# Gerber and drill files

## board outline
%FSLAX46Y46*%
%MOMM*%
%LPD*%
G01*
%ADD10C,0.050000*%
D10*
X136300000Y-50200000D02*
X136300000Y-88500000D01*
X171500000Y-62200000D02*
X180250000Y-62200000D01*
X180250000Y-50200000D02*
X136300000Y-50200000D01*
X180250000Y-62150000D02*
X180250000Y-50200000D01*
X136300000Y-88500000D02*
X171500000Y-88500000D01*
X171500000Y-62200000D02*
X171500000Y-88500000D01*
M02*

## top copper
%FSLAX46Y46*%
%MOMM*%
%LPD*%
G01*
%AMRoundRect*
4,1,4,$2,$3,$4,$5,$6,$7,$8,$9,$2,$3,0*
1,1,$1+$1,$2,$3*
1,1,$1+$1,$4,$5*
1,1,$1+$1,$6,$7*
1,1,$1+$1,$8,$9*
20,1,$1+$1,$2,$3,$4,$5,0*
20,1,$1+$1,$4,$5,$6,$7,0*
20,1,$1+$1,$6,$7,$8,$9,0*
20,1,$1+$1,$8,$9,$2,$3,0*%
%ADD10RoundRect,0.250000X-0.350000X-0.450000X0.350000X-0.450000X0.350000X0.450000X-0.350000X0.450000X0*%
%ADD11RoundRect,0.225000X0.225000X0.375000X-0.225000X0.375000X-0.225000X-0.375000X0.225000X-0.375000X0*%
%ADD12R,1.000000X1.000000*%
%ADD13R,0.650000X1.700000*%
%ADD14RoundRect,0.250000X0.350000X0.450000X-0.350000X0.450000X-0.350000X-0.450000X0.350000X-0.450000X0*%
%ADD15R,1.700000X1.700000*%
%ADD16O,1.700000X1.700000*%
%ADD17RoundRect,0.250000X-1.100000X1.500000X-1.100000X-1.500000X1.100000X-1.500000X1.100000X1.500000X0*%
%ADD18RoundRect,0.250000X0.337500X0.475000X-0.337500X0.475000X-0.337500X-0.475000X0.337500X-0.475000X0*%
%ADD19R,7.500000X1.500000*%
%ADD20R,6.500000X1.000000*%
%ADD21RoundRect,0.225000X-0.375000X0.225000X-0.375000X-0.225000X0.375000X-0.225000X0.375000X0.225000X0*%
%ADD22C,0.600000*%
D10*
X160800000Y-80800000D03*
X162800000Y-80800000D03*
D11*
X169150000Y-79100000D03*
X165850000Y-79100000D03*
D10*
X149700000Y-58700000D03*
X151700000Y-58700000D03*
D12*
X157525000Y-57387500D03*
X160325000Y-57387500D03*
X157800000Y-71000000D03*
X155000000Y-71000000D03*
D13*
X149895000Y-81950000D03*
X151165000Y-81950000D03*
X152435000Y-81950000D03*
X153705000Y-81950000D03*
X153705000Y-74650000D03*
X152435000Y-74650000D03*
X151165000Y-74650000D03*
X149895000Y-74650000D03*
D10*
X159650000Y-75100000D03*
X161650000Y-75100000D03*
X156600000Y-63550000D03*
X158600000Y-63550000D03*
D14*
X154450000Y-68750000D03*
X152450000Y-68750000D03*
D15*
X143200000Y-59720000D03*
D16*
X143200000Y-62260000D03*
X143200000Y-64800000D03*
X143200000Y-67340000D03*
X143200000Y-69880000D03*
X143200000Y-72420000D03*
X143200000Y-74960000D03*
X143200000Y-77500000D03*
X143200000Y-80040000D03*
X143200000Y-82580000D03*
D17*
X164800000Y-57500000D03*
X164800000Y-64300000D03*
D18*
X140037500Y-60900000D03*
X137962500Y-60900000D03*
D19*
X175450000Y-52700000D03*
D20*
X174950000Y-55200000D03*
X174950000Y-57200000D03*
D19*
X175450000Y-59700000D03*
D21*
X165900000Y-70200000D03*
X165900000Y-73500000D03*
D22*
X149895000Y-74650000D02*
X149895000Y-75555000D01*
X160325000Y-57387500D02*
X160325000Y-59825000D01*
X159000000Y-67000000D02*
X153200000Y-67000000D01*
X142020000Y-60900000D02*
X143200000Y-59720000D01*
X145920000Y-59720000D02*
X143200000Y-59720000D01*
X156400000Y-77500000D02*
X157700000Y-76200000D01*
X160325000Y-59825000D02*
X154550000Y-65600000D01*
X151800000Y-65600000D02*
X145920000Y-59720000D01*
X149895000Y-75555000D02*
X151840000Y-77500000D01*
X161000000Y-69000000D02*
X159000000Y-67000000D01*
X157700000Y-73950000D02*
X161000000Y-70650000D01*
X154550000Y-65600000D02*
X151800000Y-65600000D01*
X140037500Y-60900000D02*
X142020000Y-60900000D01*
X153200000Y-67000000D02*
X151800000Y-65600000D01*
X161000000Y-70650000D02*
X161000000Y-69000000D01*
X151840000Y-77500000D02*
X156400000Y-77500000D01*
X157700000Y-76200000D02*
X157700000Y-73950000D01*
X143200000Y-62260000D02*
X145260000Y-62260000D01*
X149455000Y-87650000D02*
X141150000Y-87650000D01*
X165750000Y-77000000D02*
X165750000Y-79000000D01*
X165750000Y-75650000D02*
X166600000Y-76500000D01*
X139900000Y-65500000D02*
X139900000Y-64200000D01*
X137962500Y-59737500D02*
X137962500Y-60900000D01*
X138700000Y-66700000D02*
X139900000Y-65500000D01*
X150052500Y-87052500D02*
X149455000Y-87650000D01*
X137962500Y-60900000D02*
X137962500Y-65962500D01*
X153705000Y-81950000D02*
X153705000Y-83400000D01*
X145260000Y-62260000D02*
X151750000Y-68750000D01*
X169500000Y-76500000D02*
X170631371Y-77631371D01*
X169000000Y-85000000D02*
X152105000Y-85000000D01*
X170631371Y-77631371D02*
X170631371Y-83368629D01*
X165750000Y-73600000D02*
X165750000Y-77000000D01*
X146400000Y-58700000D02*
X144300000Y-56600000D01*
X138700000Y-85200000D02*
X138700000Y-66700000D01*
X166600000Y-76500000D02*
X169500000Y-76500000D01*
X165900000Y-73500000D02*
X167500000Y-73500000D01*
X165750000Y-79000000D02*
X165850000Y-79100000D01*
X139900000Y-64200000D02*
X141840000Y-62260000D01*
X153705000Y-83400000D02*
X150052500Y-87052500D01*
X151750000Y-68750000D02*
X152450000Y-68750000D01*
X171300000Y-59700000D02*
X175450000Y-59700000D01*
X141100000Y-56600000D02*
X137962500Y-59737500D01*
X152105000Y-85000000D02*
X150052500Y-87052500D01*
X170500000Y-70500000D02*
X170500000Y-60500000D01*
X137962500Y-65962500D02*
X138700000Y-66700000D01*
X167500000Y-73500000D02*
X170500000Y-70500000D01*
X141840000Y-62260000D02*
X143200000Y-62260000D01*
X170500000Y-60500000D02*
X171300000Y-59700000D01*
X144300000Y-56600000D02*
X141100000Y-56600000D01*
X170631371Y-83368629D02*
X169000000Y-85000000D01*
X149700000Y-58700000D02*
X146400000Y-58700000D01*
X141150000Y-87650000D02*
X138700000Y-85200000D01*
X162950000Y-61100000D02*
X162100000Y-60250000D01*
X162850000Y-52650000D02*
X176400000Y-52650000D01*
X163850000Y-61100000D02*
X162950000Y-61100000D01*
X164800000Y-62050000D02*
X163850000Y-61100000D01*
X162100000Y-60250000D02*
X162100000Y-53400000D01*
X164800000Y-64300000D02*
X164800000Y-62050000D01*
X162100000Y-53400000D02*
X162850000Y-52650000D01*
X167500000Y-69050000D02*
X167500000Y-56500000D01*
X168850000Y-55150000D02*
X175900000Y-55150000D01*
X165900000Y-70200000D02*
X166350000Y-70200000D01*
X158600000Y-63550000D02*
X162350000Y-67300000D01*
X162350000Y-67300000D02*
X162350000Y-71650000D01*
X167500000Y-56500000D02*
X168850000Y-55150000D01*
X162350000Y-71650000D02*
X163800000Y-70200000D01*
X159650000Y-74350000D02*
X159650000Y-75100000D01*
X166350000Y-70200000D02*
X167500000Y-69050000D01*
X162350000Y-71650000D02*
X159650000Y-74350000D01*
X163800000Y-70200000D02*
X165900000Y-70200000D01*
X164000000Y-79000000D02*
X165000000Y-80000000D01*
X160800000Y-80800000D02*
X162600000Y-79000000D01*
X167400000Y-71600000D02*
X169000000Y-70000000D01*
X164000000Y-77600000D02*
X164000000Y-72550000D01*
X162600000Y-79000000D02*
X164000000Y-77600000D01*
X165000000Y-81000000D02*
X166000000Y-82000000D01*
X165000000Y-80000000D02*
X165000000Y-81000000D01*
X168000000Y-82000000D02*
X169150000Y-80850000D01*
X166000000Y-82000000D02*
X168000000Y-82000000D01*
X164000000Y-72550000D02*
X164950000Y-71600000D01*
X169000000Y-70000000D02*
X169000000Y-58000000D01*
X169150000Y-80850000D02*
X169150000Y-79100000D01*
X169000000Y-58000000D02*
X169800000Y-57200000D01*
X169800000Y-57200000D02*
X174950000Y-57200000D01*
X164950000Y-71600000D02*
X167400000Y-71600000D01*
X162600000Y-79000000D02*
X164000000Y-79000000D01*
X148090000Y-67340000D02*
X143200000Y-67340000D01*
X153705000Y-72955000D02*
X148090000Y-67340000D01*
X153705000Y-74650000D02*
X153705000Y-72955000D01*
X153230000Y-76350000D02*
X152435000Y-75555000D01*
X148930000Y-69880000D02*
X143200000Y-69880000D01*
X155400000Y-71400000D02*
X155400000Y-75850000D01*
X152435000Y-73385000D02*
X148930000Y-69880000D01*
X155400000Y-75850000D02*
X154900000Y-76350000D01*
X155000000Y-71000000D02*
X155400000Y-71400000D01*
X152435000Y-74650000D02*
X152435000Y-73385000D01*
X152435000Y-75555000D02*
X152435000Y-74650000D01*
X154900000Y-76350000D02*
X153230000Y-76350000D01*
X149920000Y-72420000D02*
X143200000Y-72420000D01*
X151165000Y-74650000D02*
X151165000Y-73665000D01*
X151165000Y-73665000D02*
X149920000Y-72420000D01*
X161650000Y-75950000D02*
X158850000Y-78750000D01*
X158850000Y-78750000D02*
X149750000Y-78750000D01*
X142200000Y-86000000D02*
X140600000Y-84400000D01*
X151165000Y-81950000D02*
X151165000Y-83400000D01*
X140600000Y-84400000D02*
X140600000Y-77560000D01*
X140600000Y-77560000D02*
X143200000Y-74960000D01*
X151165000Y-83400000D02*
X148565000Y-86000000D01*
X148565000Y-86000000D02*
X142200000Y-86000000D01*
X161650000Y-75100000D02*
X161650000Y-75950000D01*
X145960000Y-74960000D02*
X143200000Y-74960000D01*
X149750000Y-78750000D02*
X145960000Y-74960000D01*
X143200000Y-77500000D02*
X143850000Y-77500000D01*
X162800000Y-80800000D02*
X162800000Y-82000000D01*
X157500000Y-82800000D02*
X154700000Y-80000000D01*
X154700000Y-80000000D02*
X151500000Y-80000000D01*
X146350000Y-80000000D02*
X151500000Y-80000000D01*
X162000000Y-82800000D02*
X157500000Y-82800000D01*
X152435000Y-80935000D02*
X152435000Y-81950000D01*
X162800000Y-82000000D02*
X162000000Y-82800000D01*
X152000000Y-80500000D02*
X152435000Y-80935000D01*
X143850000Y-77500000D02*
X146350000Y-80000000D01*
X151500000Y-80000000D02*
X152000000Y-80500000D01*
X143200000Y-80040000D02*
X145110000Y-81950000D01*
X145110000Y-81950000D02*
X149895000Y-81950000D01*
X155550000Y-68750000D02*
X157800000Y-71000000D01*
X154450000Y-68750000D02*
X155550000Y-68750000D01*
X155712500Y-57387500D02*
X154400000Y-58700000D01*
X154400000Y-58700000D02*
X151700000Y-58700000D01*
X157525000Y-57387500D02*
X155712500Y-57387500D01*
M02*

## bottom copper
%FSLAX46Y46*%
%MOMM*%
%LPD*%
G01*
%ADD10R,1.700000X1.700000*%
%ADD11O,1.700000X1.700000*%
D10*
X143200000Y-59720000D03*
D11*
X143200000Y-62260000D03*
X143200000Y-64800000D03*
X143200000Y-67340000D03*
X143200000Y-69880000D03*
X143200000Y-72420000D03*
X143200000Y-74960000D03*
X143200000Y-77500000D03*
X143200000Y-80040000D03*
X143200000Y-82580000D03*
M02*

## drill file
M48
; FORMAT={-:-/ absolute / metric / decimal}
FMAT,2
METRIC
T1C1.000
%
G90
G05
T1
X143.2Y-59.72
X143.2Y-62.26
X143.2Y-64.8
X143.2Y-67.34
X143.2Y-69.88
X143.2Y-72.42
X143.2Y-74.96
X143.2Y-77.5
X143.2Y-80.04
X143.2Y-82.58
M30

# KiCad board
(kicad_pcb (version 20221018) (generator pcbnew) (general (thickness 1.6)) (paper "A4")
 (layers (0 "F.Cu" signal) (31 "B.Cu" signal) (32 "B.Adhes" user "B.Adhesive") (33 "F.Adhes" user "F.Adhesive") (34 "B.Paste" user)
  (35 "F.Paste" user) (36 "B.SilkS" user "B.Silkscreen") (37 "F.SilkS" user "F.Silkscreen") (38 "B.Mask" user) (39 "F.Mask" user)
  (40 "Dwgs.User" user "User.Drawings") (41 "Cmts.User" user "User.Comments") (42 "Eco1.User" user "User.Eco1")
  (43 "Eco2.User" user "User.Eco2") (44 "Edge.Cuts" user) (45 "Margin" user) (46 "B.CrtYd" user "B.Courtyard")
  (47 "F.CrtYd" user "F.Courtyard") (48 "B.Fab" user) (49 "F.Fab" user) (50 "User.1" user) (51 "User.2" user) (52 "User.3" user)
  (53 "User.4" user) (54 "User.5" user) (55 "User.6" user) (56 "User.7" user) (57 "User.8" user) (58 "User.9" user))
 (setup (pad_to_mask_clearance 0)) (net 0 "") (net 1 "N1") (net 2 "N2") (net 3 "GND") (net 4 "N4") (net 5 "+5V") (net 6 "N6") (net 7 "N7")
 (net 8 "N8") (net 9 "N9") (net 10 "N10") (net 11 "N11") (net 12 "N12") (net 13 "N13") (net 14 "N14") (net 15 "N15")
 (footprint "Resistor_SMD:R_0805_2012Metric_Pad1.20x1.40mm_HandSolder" (layer "F.Cu") (at 161.8 80.8)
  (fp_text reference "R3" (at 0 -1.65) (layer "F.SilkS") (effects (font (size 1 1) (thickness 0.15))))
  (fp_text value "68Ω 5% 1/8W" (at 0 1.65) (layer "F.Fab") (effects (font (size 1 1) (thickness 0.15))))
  (pad "1" smd roundrect (at -1 0) (size 1.2 1.4) (layers "F.Cu" "F.Paste" "F.Mask") (roundrect_rratio 0.208333) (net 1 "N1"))
  (pad "2" smd roundrect (at 1 0) (size 1.2 1.4) (layers "F.Cu" "F.Paste" "F.Mask") (roundrect_rratio 0.208333) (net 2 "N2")))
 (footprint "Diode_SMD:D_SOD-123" (layer "F.Cu") (at 167.5 79.1 180)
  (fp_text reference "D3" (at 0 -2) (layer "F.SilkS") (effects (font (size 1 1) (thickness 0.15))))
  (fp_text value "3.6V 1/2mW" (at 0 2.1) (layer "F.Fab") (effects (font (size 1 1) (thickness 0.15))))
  (pad "1" smd roundrect (at -1.65 0 180) (size 0.9 1.2) (layers "F.Cu" "F.Paste" "F.Mask") (roundrect_rratio 0.25) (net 1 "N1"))
  (pad "2" smd roundrect (at 1.65 0 180) (size 0.9 1.2) (layers "F.Cu" "F.Paste" "F.Mask") (roundrect_rratio 0.25) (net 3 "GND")))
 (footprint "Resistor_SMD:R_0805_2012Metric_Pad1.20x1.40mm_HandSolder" (layer "F.Cu") (at 150.7 58.7)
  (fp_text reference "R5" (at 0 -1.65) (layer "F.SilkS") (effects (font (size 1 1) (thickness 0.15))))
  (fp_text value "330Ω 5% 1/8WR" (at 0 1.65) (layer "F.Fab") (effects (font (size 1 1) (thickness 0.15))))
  (pad "1" smd roundrect (at -1 0) (size 1.2 1.4) (layers "F.Cu" "F.Paste" "F.Mask") (roundrect_rratio 0.208333) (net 3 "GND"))
  (pad "2" smd roundrect (at 1 0) (size 1.2 1.4) (layers "F.Cu" "F.Paste" "F.Mask") (roundrect_rratio 0.208333) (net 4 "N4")))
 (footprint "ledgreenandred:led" (layer "F.Cu") (at 159.325 57.3875)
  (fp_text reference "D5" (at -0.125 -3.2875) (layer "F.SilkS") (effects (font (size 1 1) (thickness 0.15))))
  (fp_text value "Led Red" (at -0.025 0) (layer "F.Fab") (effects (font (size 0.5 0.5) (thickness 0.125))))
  (pad "1" smd rect (at -1.8 0) (size 1 1) (layers "F.Cu" "F.Paste" "F.Mask") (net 4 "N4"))
  (pad "2" smd rect (at 1 0) (size 1 1) (layers "F.Cu" "F.Paste" "F.Mask") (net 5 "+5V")))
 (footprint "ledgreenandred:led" (layer "F.Cu") (at 156 71 180)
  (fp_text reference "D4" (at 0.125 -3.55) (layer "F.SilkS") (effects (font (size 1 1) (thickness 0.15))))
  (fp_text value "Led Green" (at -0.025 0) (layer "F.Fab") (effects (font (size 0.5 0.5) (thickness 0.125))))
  (pad "1" smd rect (at -1.8 0 180) (size 1 1) (layers "F.Cu" "F.Paste" "F.Mask") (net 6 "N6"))
  (pad "2" smd rect (at 1 0 180) (size 1 1) (layers "F.Cu" "F.Paste" "F.Mask") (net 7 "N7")))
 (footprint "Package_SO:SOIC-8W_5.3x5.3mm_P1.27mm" (layer "F.Cu") (at 151.8 78.3 90)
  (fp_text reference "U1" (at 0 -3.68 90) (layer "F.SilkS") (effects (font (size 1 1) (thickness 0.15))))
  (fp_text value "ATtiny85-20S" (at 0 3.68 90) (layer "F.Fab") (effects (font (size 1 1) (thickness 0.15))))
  (pad "1" smd rect (at -3.65 -1.905 90) (size 1.7 0.65) (layers "F.Cu" "F.Paste" "F.Mask") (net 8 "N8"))
  (pad "2" smd rect (at -3.65 -0.635 90) (size 1.7 0.65) (layers "F.Cu" "F.Paste" "F.Mask") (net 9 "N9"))
  (pad "3" smd rect (at -3.65 0.635 90) (size 1.7 0.65) (layers "F.Cu" "F.Paste" "F.Mask") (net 2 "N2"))
  (pad "4" smd rect (at -3.65 1.905 90) (size 1.7 0.65) (layers "F.Cu" "F.Paste" "F.Mask") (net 3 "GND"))
  (pad "5" smd rect (at 3.65 1.905 90) (size 1.7 0.65) (layers "F.Cu" "F.Paste" "F.Mask") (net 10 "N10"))
  (pad "6" smd rect (at 3.65 0.635 90) (size 1.7 0.65) (layers "F.Cu" "F.Paste" "F.Mask") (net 7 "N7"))
  (pad "7" smd rect (at 3.65 -0.635 90) (size 1.7 0.65) (layers "F.Cu" "F.Paste" "F.Mask") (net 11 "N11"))
  (pad "8" smd rect (at 3.65 -1.905 90) (size 1.7 0.65) (layers "F.Cu" "F.Paste" "F.Mask") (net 5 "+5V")))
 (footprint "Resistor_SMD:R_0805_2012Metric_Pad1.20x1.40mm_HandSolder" (layer "F.Cu") (at 160.65 75.1)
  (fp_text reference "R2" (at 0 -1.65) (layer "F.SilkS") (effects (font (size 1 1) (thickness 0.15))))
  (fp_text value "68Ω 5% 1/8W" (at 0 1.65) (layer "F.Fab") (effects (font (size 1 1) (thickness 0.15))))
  (pad "1" smd roundrect (at -1 0) (size 1.2 1.4) (layers "F.Cu" "F.Paste" "F.Mask") (roundrect_rratio 0.208333) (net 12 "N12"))
  (pad "2" smd roundrect (at 1 0) (size 1.2 1.4) (layers "F.Cu" "F.Paste" "F.Mask") (roundrect_rratio 0.208333) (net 9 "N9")))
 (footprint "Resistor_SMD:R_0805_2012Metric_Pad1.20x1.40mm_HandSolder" (layer "F.Cu") (at 157.6 63.55)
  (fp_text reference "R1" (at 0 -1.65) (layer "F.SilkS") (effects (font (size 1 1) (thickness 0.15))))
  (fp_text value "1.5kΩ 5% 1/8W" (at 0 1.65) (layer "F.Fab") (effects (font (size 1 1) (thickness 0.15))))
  (pad "1" smd roundrect (at -1 0) (size 1.2 1.4) (layers "F.Cu" "F.Paste" "F.Mask") (roundrect_rratio 0.208333) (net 5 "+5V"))
  (pad "2" smd roundrect (at 1 0) (size 1.2 1.4) (layers "F.Cu" "F.Paste" "F.Mask") (roundrect_rratio 0.208333) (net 12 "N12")))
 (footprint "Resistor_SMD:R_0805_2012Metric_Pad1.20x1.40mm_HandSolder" (layer "F.Cu") (at 153.45 68.75 180)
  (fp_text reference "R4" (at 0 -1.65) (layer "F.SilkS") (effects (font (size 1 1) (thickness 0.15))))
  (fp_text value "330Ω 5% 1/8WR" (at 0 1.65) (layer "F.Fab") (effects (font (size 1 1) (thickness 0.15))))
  (pad "1" smd roundrect (at -1 0 180) (size 1.2 1.4) (layers "F.Cu" "F.Paste" "F.Mask") (roundrect_rratio 0.208333) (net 6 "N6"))
  (pad "2" smd roundrect (at 1 0 180) (size 1.2 1.4) (layers "F.Cu" "F.Paste" "F.Mask") (roundrect_rratio 0.208333) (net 3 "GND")))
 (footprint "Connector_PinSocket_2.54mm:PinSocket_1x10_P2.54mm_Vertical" (layer "F.Cu") (at 143.2 59.72)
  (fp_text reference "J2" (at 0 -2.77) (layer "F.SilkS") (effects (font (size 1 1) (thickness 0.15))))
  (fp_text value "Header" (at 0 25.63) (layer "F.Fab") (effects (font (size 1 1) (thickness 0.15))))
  (pad "1" thru_hole rect (at 0 0) (size 1.7 1.7) (drill 1) (layers "*.Cu" "*.Mask") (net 5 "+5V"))
  (pad "2" thru_hole oval (at 0 2.54) (size 1.7 1.7) (drill 1) (layers "*.Cu" "*.Mask") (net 3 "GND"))
  (pad "3" thru_hole oval (at 0 5.08) (size 1.7 1.7) (drill 1) (layers "*.Cu" "*.Mask") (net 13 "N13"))
  (pad "4" thru_hole oval (at 0 7.62) (size 1.7 1.7) (drill 1) (layers "*.Cu" "*.Mask") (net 10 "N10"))
  (pad "5" thru_hole oval (at 0 10.16) (size 1.7 1.7) (drill 1) (layers "*.Cu" "*.Mask") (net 7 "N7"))
  (pad "6" thru_hole oval (at 0 12.7) (size 1.7 1.7) (drill 1) (layers "*.Cu" "*.Mask") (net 11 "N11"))
  (pad "7" thru_hole oval (at 0 15.24) (size 1.7 1.7) (drill 1) (layers "*.Cu" "*.Mask") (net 9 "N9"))
  (pad "8" thru_hole oval (at 0 17.78) (size 1.7 1.7) (drill 1) (layers "*.Cu" "*.Mask") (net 2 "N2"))
  (pad "9" thru_hole oval (at 0 20.32) (size 1.7 1.7) (drill 1) (layers "*.Cu" "*.Mask") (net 8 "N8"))
  (pad "10" thru_hole oval (at 0 22.86) (size 1.7 1.7) (drill 1) (layers "*.Cu" "*.Mask") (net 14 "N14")))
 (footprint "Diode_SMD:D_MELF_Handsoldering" (layer "F.Cu") (at 164.8 60.9 -90)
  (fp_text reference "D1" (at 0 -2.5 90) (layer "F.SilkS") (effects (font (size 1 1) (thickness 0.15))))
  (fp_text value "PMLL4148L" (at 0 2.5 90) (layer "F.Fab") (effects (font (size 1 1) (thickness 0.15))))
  (pad "1" smd roundrect (at -3.4 0 270) (size 3.5 2.7) (layers "F.Cu" "F.Paste" "F.Mask") (roundrect_rratio 0.0925925926) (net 5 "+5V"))
  (pad "2" smd roundrect (at 3.4 0 270) (size 3.5 2.7) (layers "F.Cu" "F.Paste" "F.Mask") (roundrect_rratio 0.0925925926) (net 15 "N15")))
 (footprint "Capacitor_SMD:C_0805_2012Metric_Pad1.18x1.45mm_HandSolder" (layer "F.Cu") (at 139 60.9 180)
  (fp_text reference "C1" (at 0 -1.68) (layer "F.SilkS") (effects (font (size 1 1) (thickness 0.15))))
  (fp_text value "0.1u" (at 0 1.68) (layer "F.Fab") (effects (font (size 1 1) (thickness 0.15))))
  (pad "1" smd roundrect (at -1.0375 0 180) (size 1.175 1.45) (layers "F.Cu" "F.Paste" "F.Mask") (roundrect_rratio 0.212766) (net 5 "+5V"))
  (pad "2" smd roundrect (at 1.0375 0 180) (size 1.175 1.45) (layers "F.Cu" "F.Paste" "F.Mask") (roundrect_rratio 0.212766) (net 3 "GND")))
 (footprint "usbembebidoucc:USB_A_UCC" (layer "F.Cu") (at 175.25 56.2 180)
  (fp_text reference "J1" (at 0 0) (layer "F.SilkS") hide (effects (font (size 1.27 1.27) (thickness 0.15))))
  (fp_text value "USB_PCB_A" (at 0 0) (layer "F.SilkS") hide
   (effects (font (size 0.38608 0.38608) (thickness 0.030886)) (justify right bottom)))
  (pad "1" smd rect (at -0.2 3.5 180) (size 7.5 1.5) (layers "F.Cu" "F.Paste" "F.Mask") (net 15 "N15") (solder_mask_margin 0.1016))
  (pad "2" smd rect (at 0.3 1 180) (size 6.5 1) (layers "F.Cu" "F.Paste" "F.Mask") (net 12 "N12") (solder_mask_margin 0.1016))
  (pad "3" smd rect (at 0.3 -1 180) (size 6.5 1) (layers "F.Cu" "F.Paste" "F.Mask") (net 1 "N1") (solder_mask_margin 0.1016))
  (pad "4" smd rect (at -0.2 -3.5 180) (size 7.5 1.5) (layers "F.Cu" "F.Paste" "F.Mask") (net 3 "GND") (solder_mask_margin 0.1016)))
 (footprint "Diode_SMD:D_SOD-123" (layer "F.Cu") (at 165.9 71.85 -90)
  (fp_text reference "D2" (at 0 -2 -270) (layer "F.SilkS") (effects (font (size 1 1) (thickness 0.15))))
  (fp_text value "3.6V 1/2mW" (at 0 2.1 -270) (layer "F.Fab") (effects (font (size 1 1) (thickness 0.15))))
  (pad "1" smd roundrect (at -1.65 0 270) (size 0.9 1.2) (layers "F.Cu" "F.Paste" "F.Mask") (roundrect_rratio 0.25) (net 12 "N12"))
  (pad "2" smd roundrect (at 1.65 0 270) (size 0.9 1.2) (layers "F.Cu" "F.Paste" "F.Mask") (roundrect_rratio 0.25) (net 3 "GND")))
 (gr_line (start 136.3 50.2) (end 136.3 88.5) (stroke (width 0.05) (type default)) (layer "Edge.Cuts"))
 (gr_line (start 171.5 62.2) (end 180.25 62.2) (stroke (width 0.05) (type default)) (layer "Edge.Cuts"))
 (gr_line (start 180.25 50.2) (end 136.3 50.2) (stroke (width 0.05) (type default)) (layer "Edge.Cuts"))
 (gr_line (start 180.25 62.15) (end 180.25 50.2) (stroke (width 0.05) (type default)) (layer "Edge.Cuts"))
 (gr_line (start 136.3 88.5) (end 171.5 88.5) (stroke (width 0.05) (type default)) (layer "Edge.Cuts"))
 (gr_line (start 171.5 62.2) (end 171.5 88.5) (stroke (width 0.05) (type default)) (layer "Edge.Cuts"))
 (segment (start 149.895 74.65) (end 149.895 75.555) (width 0.6) (layer "F.Cu") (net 5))
 (segment (start 160.325 57.3875) (end 160.325 59.825) (width 0.6) (layer "F.Cu") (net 5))
 (segment (start 159 67) (end 153.2 67) (width 0.6) (layer "F.Cu") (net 5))
 (segment (start 142.02 60.9) (end 143.2 59.72) (width 0.6) (layer "F.Cu") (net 5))
 (segment (start 145.92 59.72) (end 143.2 59.72) (width 0.6) (layer "F.Cu") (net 5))
 (segment (start 156.4 77.5) (end 157.7 76.2) (width 0.6) (layer "F.Cu") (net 5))
 (segment (start 160.325 59.825) (end 154.55 65.6) (width 0.6) (layer "F.Cu") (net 5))
 (segment (start 151.8 65.6) (end 145.92 59.72) (width 0.6) (layer "F.Cu") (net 5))
 (segment (start 149.895 75.555) (end 151.84 77.5) (width 0.6) (layer "F.Cu") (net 5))
 (segment (start 161 69) (end 159 67) (width 0.6) (layer "F.Cu") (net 5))
 (segment (start 157.7 73.95) (end 161 70.65) (width 0.6) (layer "F.Cu") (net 5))
 (segment (start 154.55 65.6) (end 151.8 65.6) (width 0.6) (layer "F.Cu") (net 5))
 (segment (start 140.0375 60.9) (end 142.02 60.9) (width 0.6) (layer "F.Cu") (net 5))
 (segment (start 153.2 67) (end 151.8 65.6) (width 0.6) (layer "F.Cu") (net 5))
 (segment (start 161 70.65) (end 161 69) (width 0.6) (layer "F.Cu") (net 5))
 (segment (start 151.84 77.5) (end 156.4 77.5) (width 0.6) (layer "F.Cu") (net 5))
 (segment (start 157.7 76.2) (end 157.7 73.95) (width 0.6) (layer "F.Cu") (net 5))
 (segment (start 143.2 62.26) (end 145.26 62.26) (width 0.6) (layer "F.Cu") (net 3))
 (segment (start 149.455 87.65) (end 141.15 87.65) (width 0.6) (layer "F.Cu") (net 3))
 (segment (start 165.75 77) (end 165.75 79) (width 0.6) (layer "F.Cu") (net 3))
 (segment (start 165.75 75.65) (end 166.6 76.5) (width 0.6) (layer "F.Cu") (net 3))
 (segment (start 139.9 65.5) (end 139.9 64.2) (width 0.6) (layer "F.Cu") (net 3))
 (segment (start 137.9625 59.7375) (end 137.9625 60.9) (width 0.6) (layer "F.Cu") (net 3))
 (segment (start 138.7 66.7) (end 139.9 65.5) (width 0.6) (layer "F.Cu") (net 3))
 (segment (start 150.0525 87.0525) (end 149.455 87.65) (width 0.6) (layer "F.Cu") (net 3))
 (segment (start 137.9625 60.9) (end 137.9625 65.9625) (width 0.6) (layer "F.Cu") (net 3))
 (segment (start 153.705 81.95) (end 153.705 83.4) (width 0.6) (layer "F.Cu") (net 3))
 (segment (start 145.26 62.26) (end 151.75 68.75) (width 0.6) (layer "F.Cu") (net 3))
 (segment (start 169.5 76.5) (end 170.631371 77.631371) (width 0.6) (layer "F.Cu") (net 3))
 (segment (start 169 85) (end 152.105 85) (width 0.6) (layer "F.Cu") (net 3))
 (segment (start 170.631371 77.631371) (end 170.631371 83.368629) (width 0.6) (layer "F.Cu") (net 3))
 (segment (start 165.75 73.6) (end 165.75 77) (width 0.6) (layer "F.Cu") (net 3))
 (segment (start 146.4 58.7) (end 144.3 56.6) (width 0.6) (layer "F.Cu") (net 3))
 (segment (start 138.7 85.2) (end 138.7 66.7) (width 0.6) (layer "F.Cu") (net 3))
 (segment (start 166.6 76.5) (end 169.5 76.5) (width 0.6) (layer "F.Cu") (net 3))
 (segment (start 165.9 73.5) (end 167.5 73.5) (width 0.6) (layer "F.Cu") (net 3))
 (segment (start 165.75 79) (end 165.85 79.1) (width 0.6) (layer "F.Cu") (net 3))
 (segment (start 139.9 64.2) (end 141.84 62.26) (width 0.6) (layer "F.Cu") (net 3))
 (segment (start 153.705 83.4) (end 150.0525 87.0525) (width 0.6) (layer "F.Cu") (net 3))
 (segment (start 151.75 68.75) (end 152.45 68.75) (width 0.6) (layer "F.Cu") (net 3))
 (segment (start 171.3 59.7) (end 175.45 59.7) (width 0.6) (layer "F.Cu") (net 3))
 (segment (start 141.1 56.6) (end 137.9625 59.7375) (width 0.6) (layer "F.Cu") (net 3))
 (segment (start 152.105 85) (end 150.0525 87.0525) (width 0.6) (layer "F.Cu") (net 3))
 (segment (start 170.5 70.5) (end 170.5 60.5) (width 0.6) (layer "F.Cu") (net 3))
 (segment (start 137.9625 65.9625) (end 138.7 66.7) (width 0.6) (layer "F.Cu") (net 3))
 (segment (start 167.5 73.5) (end 170.5 70.5) (width 0.6) (layer "F.Cu") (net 3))
 (segment (start 141.84 62.26) (end 143.2 62.26) (width 0.6) (layer "F.Cu") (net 3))
 (segment (start 170.5 60.5) (end 171.3 59.7) (width 0.6) (layer "F.Cu") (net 3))
 (segment (start 144.3 56.6) (end 141.1 56.6) (width 0.6) (layer "F.Cu") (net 3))
 (segment (start 170.631371 83.368629) (end 169 85) (width 0.6) (layer "F.Cu") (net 3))
 (segment (start 149.7 58.7) (end 146.4 58.7) (width 0.6) (layer "F.Cu") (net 3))
 (segment (start 141.15 87.65) (end 138.7 85.2) (width 0.6) (layer "F.Cu") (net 3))
 (segment (start 162.95 61.1) (end 162.1 60.25) (width 0.6) (layer "F.Cu") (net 15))
 (segment (start 162.85 52.65) (end 176.4 52.65) (width 0.6) (layer "F.Cu") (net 15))
 (segment (start 163.85 61.1) (end 162.95 61.1) (width 0.6) (layer "F.Cu") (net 15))
 (segment (start 164.8 62.05) (end 163.85 61.1) (width 0.6) (layer "F.Cu") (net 15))
 (segment (start 162.1 60.25) (end 162.1 53.4) (width 0.6) (layer "F.Cu") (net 15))
 (segment (start 164.8 64.3) (end 164.8 62.05) (width 0.6) (layer "F.Cu") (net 15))
 (segment (start 162.1 53.4) (end 162.85 52.65) (width 0.6) (layer "F.Cu") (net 15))
 (segment (start 167.5 69.05) (end 167.5 56.5) (width 0.6) (layer "F.Cu") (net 12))
 (segment (start 168.85 55.15) (end 175.9 55.15) (width 0.6) (layer "F.Cu") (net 12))
 (segment (start 165.9 70.2) (end 166.35 70.2) (width 0.6) (layer "F.Cu") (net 12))
 (segment (start 158.6 63.55) (end 162.35 67.3) (width 0.6) (layer "F.Cu") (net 12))
 (segment (start 162.35 67.3) (end 162.35 71.65) (width 0.6) (layer "F.Cu") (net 12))
 (segment (start 167.5 56.5) (end 168.85 55.15) (width 0.6) (layer "F.Cu") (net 12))
 (segment (start 162.35 71.65) (end 163.8 70.2) (width 0.6) (layer "F.Cu") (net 12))
 (segment (start 159.65 74.35) (end 159.65 75.1) (width 0.6) (layer "F.Cu") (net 12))
 (segment (start 166.35 70.2) (end 167.5 69.05) (width 0.6) (layer "F.Cu") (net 12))
 (segment (start 162.35 71.65) (end 159.65 74.35) (width 0.6) (layer "F.Cu") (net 12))
 (segment (start 163.8 70.2) (end 165.9 70.2) (width 0.6) (layer "F.Cu") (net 12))
 (segment (start 164 79) (end 165 80) (width 0.6) (layer "F.Cu") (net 1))
 (segment (start 160.8 80.8) (end 162.6 79) (width 0.6) (layer "F.Cu") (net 1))
 (segment (start 167.4 71.6) (end 169 70) (width 0.6) (layer "F.Cu") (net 1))
 (segment (start 164 77.6) (end 164 72.55) (width 0.6) (layer "F.Cu") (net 1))
 (segment (start 162.6 79) (end 164 77.6) (width 0.6) (layer "F.Cu") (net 1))
 (segment (start 165 81) (end 166 82) (width 0.6) (layer "F.Cu") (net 1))
 (segment (start 165 80) (end 165 81) (width 0.6) (layer "F.Cu") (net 1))
 (segment (start 168 82) (end 169.15 80.85) (width 0.6) (layer "F.Cu") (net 1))
 (segment (start 166 82) (end 168 82) (width 0.6) (layer "F.Cu") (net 1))
 (segment (start 164 72.55) (end 164.95 71.6) (width 0.6) (layer "F.Cu") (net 1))
 (segment (start 169 70) (end 169 58) (width 0.6) (layer "F.Cu") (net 1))
 (segment (start 169.15 80.85) (end 169.15 79.1) (width 0.6) (layer "F.Cu") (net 1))
 (segment (start 169 58) (end 169.8 57.2) (width 0.6) (layer "F.Cu") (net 1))
 (segment (start 169.8 57.2) (end 174.95 57.2) (width 0.6) (layer "F.Cu") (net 1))
 (segment (start 164.95 71.6) (end 167.4 71.6) (width 0.6) (layer "F.Cu") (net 1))
 (segment (start 162.6 79) (end 164 79) (width 0.6) (layer "F.Cu") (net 1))
 (segment (start 148.09 67.34) (end 143.2 67.34) (width 0.6) (layer "F.Cu") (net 10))
 (segment (start 153.705 72.955) (end 148.09 67.34) (width 0.6) (layer "F.Cu") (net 10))
 (segment (start 153.705 74.65) (end 153.705 72.955) (width 0.6) (layer "F.Cu") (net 10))
 (segment (start 153.23 76.35) (end 152.435 75.555) (width 0.6) (layer "F.Cu") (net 7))
 (segment (start 148.93 69.88) (end 143.2 69.88) (width 0.6) (layer "F.Cu") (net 7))
 (segment (start 155.4 71.4) (end 155.4 75.85) (width 0.6) (layer "F.Cu") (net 7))
 (segment (start 152.435 73.385) (end 148.93 69.88) (width 0.6) (layer "F.Cu") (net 7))
 (segment (start 155.4 75.85) (end 154.9 76.35) (width 0.6) (layer "F.Cu") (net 7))
 (segment (start 155 71) (end 155.4 71.4) (width 0.6) (layer "F.Cu") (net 7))
 (segment (start 152.435 74.65) (end 152.435 73.385) (width 0.6) (layer "F.Cu") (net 7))
 (segment (start 152.435 75.555) (end 152.435 74.65) (width 0.6) (layer "F.Cu") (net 7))
 (segment (start 154.9 76.35) (end 153.23 76.35) (width 0.6) (layer "F.Cu") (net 7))
 (segment (start 149.92 72.42) (end 143.2 72.42) (width 0.6) (layer "F.Cu") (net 11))
 (segment (start 151.165 74.65) (end 151.165 73.665) (width 0.6) (layer "F.Cu") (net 11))
 (segment (start 151.165 73.665) (end 149.92 72.42) (width 0.6) (layer "F.Cu") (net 11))
 (segment (start 161.65 75.95) (end 158.85 78.75) (width 0.6) (layer "F.Cu") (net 9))
 (segment (start 158.85 78.75) (end 149.75 78.75) (width 0.6) (layer "F.Cu") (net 9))
 (segment (start 142.2 86) (end 140.6 84.4) (width 0.6) (layer "F.Cu") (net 9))
 (segment (start 151.165 81.95) (end 151.165 83.4) (width 0.6) (layer "F.Cu") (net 9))
 (segment (start 140.6 84.4) (end 140.6 77.56) (width 0.6) (layer "F.Cu") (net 9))
 (segment (start 140.6 77.56) (end 143.2 74.96) (width 0.6) (layer "F.Cu") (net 9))
 (segment (start 151.165 83.4) (end 148.565 86) (width 0.6) (layer "F.Cu") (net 9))
 (segment (start 148.565 86) (end 142.2 86) (width 0.6) (layer "F.Cu") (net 9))
 (segment (start 161.65 75.1) (end 161.65 75.95) (width 0.6) (layer "F.Cu") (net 9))
 (segment (start 145.96 74.96) (end 143.2 74.96) (width 0.6) (layer "F.Cu") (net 9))
 (segment (start 149.75 78.75) (end 145.96 74.96) (width 0.6) (layer "F.Cu") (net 9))
 (segment (start 143.2 77.5) (end 143.85 77.5) (width 0.6) (layer "F.Cu") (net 2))
 (segment (start 162.8 80.8) (end 162.8 82) (width 0.6) (layer "F.Cu") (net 2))
 (segment (start 157.5 82.8) (end 154.7 80) (width 0.6) (layer "F.Cu") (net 2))
 (segment (start 154.7 80) (end 151.5 80) (width 0.6) (layer "F.Cu") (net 2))
 (segment (start 146.35 80) (end 151.5 80) (width 0.6) (layer "F.Cu") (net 2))
 (segment (start 162 82.8) (end 157.5 82.8) (width 0.6) (layer "F.Cu") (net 2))
 (segment (start 152.435 80.935) (end 152.435 81.95) (width 0.6) (layer "F.Cu") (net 2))
 (segment (start 162.8 82) (end 162 82.8) (width 0.6) (layer "F.Cu") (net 2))
 (segment (start 152 80.5) (end 152.435 80.935) (width 0.6) (layer "F.Cu") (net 2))
 (segment (start 143.85 77.5) (end 146.35 80) (width 0.6) (layer "F.Cu") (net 2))
 (segment (start 151.5 80) (end 152 80.5) (width 0.6) (layer "F.Cu") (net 2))
 (segment (start 143.2 80.04) (end 145.11 81.95) (width 0.6) (layer "F.Cu") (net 8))
 (segment (start 145.11 81.95) (end 149.895 81.95) (width 0.6) (layer "F.Cu") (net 8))
 (segment (start 155.55 68.75) (end 157.8 71) (width 0.6) (layer "F.Cu") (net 6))
 (segment (start 154.45 68.75) (end 155.55 68.75) (width 0.6) (layer "F.Cu") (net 6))
 (segment (start 155.7125 57.3875) (end 154.4 58.7) (width 0.6) (layer "F.Cu") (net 4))
 (segment (start 154.4 58.7) (end 151.7 58.7) (width 0.6) (layer "F.Cu") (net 4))
 (segment (start 157.525 57.3875) (end 155.7125 57.3875) (width 0.6) (layer "F.Cu") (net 4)))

